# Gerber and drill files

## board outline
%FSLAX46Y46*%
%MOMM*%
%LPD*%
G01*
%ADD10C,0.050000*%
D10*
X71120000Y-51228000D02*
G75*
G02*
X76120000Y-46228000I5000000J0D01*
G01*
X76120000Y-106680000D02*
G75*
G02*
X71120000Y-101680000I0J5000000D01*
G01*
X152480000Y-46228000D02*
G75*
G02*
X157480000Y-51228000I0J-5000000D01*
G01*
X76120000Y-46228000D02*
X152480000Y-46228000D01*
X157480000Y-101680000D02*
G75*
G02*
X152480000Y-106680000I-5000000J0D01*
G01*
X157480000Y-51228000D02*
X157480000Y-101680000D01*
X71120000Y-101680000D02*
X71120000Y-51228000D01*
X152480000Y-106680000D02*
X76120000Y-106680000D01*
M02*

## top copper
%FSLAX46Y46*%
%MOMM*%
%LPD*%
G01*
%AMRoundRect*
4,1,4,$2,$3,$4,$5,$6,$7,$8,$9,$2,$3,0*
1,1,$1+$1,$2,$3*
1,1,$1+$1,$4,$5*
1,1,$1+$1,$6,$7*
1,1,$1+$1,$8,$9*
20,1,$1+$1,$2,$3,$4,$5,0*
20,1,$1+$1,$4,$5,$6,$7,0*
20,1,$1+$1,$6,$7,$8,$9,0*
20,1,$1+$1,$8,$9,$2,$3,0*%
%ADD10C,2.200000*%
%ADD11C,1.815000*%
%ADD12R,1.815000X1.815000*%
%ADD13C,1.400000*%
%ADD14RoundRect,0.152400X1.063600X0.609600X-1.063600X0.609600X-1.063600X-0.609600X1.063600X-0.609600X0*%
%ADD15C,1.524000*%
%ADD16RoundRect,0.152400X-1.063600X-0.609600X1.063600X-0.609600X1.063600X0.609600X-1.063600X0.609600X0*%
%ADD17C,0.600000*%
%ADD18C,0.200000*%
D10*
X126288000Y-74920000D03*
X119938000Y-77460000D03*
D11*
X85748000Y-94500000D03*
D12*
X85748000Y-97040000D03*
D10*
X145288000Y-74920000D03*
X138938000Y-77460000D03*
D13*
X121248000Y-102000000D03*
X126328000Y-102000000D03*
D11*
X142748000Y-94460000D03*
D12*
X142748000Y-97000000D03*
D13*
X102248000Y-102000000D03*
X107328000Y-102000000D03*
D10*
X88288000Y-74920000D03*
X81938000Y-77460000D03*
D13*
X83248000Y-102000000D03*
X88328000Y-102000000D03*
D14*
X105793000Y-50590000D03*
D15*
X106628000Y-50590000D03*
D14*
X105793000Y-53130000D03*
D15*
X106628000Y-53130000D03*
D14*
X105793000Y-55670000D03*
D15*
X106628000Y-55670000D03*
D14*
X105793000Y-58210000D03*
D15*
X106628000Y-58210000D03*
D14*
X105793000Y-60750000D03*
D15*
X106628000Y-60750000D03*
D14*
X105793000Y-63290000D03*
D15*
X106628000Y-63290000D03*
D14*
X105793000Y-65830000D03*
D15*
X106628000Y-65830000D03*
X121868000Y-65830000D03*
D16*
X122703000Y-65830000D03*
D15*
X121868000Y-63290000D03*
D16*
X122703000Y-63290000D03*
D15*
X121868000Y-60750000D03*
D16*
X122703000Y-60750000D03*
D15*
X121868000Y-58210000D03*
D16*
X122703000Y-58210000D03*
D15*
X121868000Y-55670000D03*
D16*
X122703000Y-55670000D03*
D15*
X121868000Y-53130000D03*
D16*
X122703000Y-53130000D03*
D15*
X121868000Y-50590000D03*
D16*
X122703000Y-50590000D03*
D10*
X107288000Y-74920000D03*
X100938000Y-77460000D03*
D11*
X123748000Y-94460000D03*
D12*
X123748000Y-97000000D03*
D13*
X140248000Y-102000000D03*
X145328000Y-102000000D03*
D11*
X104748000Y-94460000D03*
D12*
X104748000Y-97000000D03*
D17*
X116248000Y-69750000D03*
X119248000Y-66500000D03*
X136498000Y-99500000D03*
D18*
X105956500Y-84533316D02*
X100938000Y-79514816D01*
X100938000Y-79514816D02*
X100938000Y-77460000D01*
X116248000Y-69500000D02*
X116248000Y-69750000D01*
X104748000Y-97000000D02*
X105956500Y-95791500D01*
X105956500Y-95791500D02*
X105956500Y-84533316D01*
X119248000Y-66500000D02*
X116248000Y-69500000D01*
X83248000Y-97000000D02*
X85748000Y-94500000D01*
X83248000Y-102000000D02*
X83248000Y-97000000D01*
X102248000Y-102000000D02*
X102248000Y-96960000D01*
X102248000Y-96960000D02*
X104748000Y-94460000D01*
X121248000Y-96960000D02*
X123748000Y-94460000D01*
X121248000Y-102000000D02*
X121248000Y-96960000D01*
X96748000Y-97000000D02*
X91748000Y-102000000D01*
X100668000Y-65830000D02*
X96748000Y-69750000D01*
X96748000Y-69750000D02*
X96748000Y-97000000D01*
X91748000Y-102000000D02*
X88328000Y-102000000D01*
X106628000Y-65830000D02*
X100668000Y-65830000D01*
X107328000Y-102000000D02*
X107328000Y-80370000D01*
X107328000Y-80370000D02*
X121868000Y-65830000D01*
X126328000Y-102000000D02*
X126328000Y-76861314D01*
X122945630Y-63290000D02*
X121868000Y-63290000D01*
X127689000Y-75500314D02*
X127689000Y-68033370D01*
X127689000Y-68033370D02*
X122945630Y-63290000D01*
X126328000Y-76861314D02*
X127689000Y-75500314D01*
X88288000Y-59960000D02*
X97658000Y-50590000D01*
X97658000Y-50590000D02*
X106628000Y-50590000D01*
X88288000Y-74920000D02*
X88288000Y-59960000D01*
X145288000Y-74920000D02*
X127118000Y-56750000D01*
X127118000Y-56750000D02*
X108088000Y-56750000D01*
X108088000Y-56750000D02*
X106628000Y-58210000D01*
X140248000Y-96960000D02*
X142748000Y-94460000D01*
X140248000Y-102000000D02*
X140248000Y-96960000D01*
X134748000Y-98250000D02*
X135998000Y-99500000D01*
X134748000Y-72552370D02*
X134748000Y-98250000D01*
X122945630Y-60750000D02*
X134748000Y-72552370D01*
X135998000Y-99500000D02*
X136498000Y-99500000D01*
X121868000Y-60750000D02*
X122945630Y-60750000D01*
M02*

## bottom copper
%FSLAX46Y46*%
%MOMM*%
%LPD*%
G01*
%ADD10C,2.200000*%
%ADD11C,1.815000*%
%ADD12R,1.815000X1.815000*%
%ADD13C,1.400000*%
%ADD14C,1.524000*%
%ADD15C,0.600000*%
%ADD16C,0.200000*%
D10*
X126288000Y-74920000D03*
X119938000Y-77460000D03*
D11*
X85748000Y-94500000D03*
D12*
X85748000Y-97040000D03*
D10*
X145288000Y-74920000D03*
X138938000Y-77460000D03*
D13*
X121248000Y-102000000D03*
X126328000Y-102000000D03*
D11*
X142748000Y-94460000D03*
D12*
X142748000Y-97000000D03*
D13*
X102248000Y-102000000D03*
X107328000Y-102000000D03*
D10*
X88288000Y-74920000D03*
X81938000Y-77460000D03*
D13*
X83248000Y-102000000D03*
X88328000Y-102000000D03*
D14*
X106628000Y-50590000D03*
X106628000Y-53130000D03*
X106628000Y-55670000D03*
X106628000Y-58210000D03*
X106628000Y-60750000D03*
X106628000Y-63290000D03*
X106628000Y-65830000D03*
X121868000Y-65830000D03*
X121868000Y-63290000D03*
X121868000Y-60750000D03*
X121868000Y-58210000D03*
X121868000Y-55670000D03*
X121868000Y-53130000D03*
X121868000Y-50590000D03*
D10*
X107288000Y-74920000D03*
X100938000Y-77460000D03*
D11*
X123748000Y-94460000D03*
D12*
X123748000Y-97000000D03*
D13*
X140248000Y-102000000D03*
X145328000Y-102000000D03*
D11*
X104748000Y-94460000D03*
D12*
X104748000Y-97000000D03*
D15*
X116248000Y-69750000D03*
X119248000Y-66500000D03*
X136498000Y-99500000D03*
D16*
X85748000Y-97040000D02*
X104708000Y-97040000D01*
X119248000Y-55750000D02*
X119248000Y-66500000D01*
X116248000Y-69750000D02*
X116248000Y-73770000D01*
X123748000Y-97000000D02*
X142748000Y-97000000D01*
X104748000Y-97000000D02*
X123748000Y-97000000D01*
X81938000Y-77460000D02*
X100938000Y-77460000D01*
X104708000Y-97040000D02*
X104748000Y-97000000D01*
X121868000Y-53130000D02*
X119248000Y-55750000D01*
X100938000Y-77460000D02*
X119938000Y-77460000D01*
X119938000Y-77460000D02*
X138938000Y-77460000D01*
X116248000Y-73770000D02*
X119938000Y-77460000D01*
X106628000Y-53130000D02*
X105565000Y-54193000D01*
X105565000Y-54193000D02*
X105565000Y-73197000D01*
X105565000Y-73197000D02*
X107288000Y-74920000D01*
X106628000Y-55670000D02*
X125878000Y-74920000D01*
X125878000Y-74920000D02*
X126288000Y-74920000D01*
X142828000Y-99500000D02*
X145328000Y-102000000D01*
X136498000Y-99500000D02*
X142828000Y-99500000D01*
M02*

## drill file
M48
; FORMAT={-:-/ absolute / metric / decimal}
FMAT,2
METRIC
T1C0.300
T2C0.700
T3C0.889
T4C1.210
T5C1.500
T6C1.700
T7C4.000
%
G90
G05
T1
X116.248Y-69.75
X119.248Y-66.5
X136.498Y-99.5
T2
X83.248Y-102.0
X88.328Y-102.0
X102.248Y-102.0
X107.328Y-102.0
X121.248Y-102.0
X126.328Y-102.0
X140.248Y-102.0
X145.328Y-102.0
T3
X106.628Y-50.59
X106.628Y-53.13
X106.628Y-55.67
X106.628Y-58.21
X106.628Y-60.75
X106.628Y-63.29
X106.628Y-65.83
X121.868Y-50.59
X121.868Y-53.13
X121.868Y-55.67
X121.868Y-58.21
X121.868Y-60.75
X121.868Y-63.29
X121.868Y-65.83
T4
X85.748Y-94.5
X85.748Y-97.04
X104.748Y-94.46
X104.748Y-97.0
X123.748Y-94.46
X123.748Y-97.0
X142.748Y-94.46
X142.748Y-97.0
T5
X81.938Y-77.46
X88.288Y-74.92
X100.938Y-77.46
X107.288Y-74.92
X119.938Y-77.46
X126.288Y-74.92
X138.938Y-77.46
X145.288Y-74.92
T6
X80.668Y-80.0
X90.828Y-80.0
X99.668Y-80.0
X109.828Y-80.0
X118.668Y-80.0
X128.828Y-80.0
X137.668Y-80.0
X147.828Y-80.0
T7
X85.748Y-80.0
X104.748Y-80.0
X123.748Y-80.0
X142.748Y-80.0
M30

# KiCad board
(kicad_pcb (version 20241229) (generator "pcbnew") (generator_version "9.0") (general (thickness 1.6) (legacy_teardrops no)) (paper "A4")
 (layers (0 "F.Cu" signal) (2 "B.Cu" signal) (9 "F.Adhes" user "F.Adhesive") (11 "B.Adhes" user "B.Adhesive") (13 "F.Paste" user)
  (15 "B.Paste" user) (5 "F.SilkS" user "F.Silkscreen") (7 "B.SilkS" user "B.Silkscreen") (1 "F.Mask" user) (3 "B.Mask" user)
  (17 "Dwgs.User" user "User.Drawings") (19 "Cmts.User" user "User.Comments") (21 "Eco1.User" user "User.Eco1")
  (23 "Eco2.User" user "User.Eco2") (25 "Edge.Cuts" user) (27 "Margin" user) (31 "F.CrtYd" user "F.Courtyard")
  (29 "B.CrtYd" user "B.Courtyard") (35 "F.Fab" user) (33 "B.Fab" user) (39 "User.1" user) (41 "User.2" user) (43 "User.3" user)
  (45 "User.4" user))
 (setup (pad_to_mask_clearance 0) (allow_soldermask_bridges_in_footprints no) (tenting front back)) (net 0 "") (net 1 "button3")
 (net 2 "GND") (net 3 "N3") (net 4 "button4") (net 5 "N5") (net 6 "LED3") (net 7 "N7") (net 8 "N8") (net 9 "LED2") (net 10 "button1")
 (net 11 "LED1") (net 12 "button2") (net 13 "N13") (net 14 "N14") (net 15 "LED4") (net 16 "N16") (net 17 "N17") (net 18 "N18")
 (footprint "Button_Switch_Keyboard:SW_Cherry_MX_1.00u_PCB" (layer "F.Cu") (at 126.288 74.92)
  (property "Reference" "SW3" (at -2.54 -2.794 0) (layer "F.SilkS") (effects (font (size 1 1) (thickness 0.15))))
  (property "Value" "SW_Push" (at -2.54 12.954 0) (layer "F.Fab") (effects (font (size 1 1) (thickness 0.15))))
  (pad "" np_thru_hole circle (at -7.62 5.08) (size 1.7 1.7) (drill 1.7) (layers "*.Cu" "*.Mask"))
  (pad "" np_thru_hole circle (at -2.54 5.08) (size 4 4) (drill 4) (layers "*.Cu" "*.Mask"))
  (pad "" np_thru_hole circle (at 2.54 5.08) (size 1.7 1.7) (drill 1.7) (layers "*.Cu" "*.Mask"))
  (pad "1" thru_hole circle (at 0 0) (size 2.2 2.2) (drill 1.5) (layers "*.Cu" "*.Mask") (remove_unused_layers no) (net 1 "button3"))
  (pad "2" thru_hole circle (at -6.35 2.54) (size 2.2 2.2) (drill 1.5) (layers "*.Cu" "*.Mask") (remove_unused_layers no) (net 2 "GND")))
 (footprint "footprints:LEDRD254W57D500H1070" (layer "F.Cu") (at 85.748 95.77 90)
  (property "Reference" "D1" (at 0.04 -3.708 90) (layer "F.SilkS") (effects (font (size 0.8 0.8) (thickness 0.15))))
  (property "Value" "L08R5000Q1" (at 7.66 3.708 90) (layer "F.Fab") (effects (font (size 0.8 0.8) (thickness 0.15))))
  (pad "A" thru_hole circle (at 1.27 0 90) (size 1.815 1.815) (drill 1.21) (layers "*.Cu" "*.Mask") (remove_unused_layers no) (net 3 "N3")
   (solder_mask_margin 0.102))
  (pad "C" thru_hole rect (at -1.27 0 90) (size 1.815 1.815) (drill 1.21) (layers "*.Cu" "*.Mask") (remove_unused_layers no) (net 2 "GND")
   (solder_mask_margin 0.102)))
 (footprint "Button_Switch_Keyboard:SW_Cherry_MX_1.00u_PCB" (layer "F.Cu") (at 145.288 74.92)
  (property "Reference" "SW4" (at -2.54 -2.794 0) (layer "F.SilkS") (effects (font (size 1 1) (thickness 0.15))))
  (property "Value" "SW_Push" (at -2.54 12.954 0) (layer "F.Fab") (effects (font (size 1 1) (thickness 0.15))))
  (pad "" np_thru_hole circle (at -7.62 5.08) (size 1.7 1.7) (drill 1.7) (layers "*.Cu" "*.Mask"))
  (pad "" np_thru_hole circle (at -2.54 5.08) (size 4 4) (drill 4) (layers "*.Cu" "*.Mask"))
  (pad "" np_thru_hole circle (at 2.54 5.08) (size 1.7 1.7) (drill 1.7) (layers "*.Cu" "*.Mask"))
  (pad "1" thru_hole circle (at 0 0) (size 2.2 2.2) (drill 1.5) (layers "*.Cu" "*.Mask") (remove_unused_layers no) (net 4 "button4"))
  (pad "2" thru_hole circle (at -6.35 2.54) (size 2.2 2.2) (drill 1.5) (layers "*.Cu" "*.Mask") (remove_unused_layers no) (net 2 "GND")))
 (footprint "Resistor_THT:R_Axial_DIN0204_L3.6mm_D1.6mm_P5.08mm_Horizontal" (layer "F.Cu") (at 121.248 102)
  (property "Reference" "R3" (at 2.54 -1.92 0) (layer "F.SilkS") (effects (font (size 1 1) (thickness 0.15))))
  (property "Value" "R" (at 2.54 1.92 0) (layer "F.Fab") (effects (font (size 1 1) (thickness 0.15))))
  (pad "1" thru_hole circle (at 0 0) (size 1.4 1.4) (drill 0.7) (layers "*.Cu" "*.Mask") (remove_unused_layers no) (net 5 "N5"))
  (pad "2" thru_hole circle (at 5.08 0) (size 1.4 1.4) (drill 0.7) (layers "*.Cu" "*.Mask") (remove_unused_layers no) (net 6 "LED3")))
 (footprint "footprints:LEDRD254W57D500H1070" (layer "F.Cu") (at 142.748 95.73 90)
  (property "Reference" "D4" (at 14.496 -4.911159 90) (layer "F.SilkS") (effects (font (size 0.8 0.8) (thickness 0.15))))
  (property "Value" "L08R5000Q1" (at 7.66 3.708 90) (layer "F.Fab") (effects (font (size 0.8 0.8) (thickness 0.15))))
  (pad "A" thru_hole circle (at 1.27 0 90) (size 1.815 1.815) (drill 1.21) (layers "*.Cu" "*.Mask") (remove_unused_layers no) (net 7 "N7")
   (solder_mask_margin 0.102))
  (pad "C" thru_hole rect (at -1.27 0 90) (size 1.815 1.815) (drill 1.21) (layers "*.Cu" "*.Mask") (remove_unused_layers no) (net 2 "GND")
   (solder_mask_margin 0.102)))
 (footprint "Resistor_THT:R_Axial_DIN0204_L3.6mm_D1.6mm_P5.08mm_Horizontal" (layer "F.Cu") (at 102.248 102)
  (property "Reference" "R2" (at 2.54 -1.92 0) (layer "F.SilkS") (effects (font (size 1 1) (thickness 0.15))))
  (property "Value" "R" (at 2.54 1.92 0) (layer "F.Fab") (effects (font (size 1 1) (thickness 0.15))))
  (pad "1" thru_hole circle (at 0 0) (size 1.4 1.4) (drill 0.7) (layers "*.Cu" "*.Mask") (remove_unused_layers no) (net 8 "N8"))
  (pad "2" thru_hole circle (at 5.08 0) (size 1.4 1.4) (drill 0.7) (layers "*.Cu" "*.Mask") (remove_unused_layers no) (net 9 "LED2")))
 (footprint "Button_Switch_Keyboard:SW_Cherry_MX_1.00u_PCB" (layer "F.Cu") (at 88.288 74.92)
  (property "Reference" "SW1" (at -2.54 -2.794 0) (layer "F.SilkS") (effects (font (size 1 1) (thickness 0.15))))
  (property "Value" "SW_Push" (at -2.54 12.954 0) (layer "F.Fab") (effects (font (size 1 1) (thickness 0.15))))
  (pad "" np_thru_hole circle (at -7.62 5.08) (size 1.7 1.7) (drill 1.7) (layers "*.Cu" "*.Mask"))
  (pad "" np_thru_hole circle (at -2.54 5.08) (size 4 4) (drill 4) (layers "*.Cu" "*.Mask"))
  (pad "" np_thru_hole circle (at 2.54 5.08) (size 1.7 1.7) (drill 1.7) (layers "*.Cu" "*.Mask"))
  (pad "1" thru_hole circle (at 0 0) (size 2.2 2.2) (drill 1.5) (layers "*.Cu" "*.Mask") (remove_unused_layers no) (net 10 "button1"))
  (pad "2" thru_hole circle (at -6.35 2.54) (size 2.2 2.2) (drill 1.5) (layers "*.Cu" "*.Mask") (remove_unused_layers no) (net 2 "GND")))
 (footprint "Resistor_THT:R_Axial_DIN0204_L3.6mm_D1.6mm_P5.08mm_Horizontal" (layer "F.Cu") (at 83.248 102)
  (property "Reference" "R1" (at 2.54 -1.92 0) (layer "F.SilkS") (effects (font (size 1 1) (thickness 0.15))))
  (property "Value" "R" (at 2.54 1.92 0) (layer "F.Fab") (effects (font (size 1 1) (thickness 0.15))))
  (pad "1" thru_hole circle (at 0 0) (size 1.4 1.4) (drill 0.7) (layers "*.Cu" "*.Mask") (remove_unused_layers no) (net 3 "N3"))
  (pad "2" thru_hole circle (at 5.08 0) (size 1.4 1.4) (drill 0.7) (layers "*.Cu" "*.Mask") (remove_unused_layers no) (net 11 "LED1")))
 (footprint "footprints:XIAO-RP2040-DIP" (layer "F.Cu") (at 114.248 58.21)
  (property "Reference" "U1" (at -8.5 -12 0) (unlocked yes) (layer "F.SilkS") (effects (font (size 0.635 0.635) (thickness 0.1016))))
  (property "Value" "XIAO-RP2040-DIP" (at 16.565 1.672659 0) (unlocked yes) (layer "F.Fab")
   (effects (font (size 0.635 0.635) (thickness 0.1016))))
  (pad "1" smd roundrect (at -8.455 -7.62 180) (size 2.432 1.524) (layers "F.Cu" "F.Mask") (roundrect_rratio 0.1) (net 10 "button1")
   (thermal_bridge_angle 45))
  (pad "1" thru_hole circle (at -7.62 -7.62 180) (size 1.524 1.524) (drill 0.889) (layers "*.Cu" "*.Mask") (remove_unused_layers no)
   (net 10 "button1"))
  (pad "2" smd roundrect (at -8.455 -5.08 180) (size 2.432 1.524) (layers "F.Cu" "F.Mask") (roundrect_rratio 0.1) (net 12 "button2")
   (thermal_bridge_angle 45))
  (pad "2" thru_hole circle (at -7.62 -5.08 180) (size 1.524 1.524) (drill 0.889) (layers "*.Cu" "*.Mask") (remove_unused_layers no)
   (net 12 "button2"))
  (pad "3" smd roundrect (at -8.455 -2.54 180) (size 2.432 1.524) (layers "F.Cu" "F.Mask") (roundrect_rratio 0.1) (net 1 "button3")
   (thermal_bridge_angle 45))
  (pad "3" thru_hole circle (at -7.62 -2.54 180) (size 1.524 1.524) (drill 0.889) (layers "*.Cu" "*.Mask") (remove_unused_layers no)
   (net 1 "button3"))
  (pad "4" smd roundrect (at -8.455 0 180) (size 2.432 1.524) (layers "F.Cu" "F.Mask") (roundrect_rratio 0.1) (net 4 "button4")
   (thermal_bridge_angle 45))
  (pad "4" thru_hole circle (at -7.62 0 180) (size 1.524 1.524) (drill 0.889) (layers "*.Cu" "*.Mask") (remove_unused_layers no)
   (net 4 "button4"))
  (pad "5" smd roundrect (at -8.455 2.54 180) (size 2.432 1.524) (layers "F.Cu" "F.Mask") (roundrect_rratio 0.1) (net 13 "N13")
   (thermal_bridge_angle 45))
  (pad "5" thru_hole circle (at -7.62 2.54 180) (size 1.524 1.524) (drill 0.889) (layers "*.Cu" "*.Mask") (remove_unused_layers no)
   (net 13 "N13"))
  (pad "6" smd roundrect (at -8.455 5.08 180) (size 2.432 1.524) (layers "F.Cu" "F.Mask") (roundrect_rratio 0.1) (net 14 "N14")
   (thermal_bridge_angle 45))
  (pad "6" thru_hole circle (at -7.62 5.08 180) (size 1.524 1.524) (drill 0.889) (layers "*.Cu" "*.Mask") (remove_unused_layers no)
   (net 14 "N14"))
  (pad "7" smd roundrect (at -8.455 7.62 180) (size 2.432 1.524) (layers "F.Cu" "F.Mask") (roundrect_rratio 0.1) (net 11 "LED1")
   (thermal_bridge_angle 45))
  (pad "7" thru_hole circle (at -7.62 7.62 180) (size 1.524 1.524) (drill 0.889) (layers "*.Cu" "*.Mask") (remove_unused_layers no)
   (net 11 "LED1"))
  (pad "8" thru_hole circle (at 7.62 7.62) (size 1.524 1.524) (drill 0.889) (layers "*.Cu" "*.Mask") (remove_unused_layers no)
   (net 9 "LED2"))
  (pad "8" smd roundrect (at 8.455 7.62) (size 2.432 1.524) (layers "F.Cu" "F.Mask") (roundrect_rratio 0.1) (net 9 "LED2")
   (thermal_bridge_angle 45))
  (pad "9" thru_hole circle (at 7.62 5.08) (size 1.524 1.524) (drill 0.889) (layers "*.Cu" "*.Mask") (remove_unused_layers no)
   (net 6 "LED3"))
  (pad "9" smd roundrect (at 8.455 5.08) (size 2.432 1.524) (layers "F.Cu" "F.Mask") (roundrect_rratio 0.1) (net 6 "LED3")
   (thermal_bridge_angle 45))
  (pad "10" thru_hole circle (at 7.62 2.54) (size 1.524 1.524) (drill 0.889) (layers "*.Cu" "*.Mask") (remove_unused_layers no)
   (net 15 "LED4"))
  (pad "10" smd roundrect (at 8.455 2.54) (size 2.432 1.524) (layers "F.Cu" "F.Mask") (roundrect_rratio 0.1) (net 15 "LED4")
   (thermal_bridge_angle 45))
  (pad "11" thru_hole circle (at 7.62 0) (size 1.524 1.524) (drill 0.889) (layers "*.Cu" "*.Mask") (remove_unused_layers no) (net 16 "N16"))
  (pad "11" smd roundrect (at 8.455 0) (size 2.432 1.524) (layers "F.Cu" "F.Mask") (roundrect_rratio 0.1) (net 16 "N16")
   (thermal_bridge_angle 45))
  (pad "12" thru_hole circle (at 7.62 -2.54) (size 1.524 1.524) (drill 0.889) (layers "*.Cu" "*.Mask") (remove_unused_layers no)
   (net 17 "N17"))
  (pad "12" smd roundrect (at 8.455 -2.54) (size 2.432 1.524) (layers "F.Cu" "F.Mask") (roundrect_rratio 0.1) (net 17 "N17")
   (thermal_bridge_angle 45))
  (pad "13" thru_hole circle (at 7.62 -5.08) (size 1.524 1.524) (drill 0.889) (layers "*.Cu" "*.Mask") (remove_unused_layers no)
   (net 2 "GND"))
  (pad "13" smd roundrect (at 8.455 -5.08) (size 2.432 1.524) (layers "F.Cu" "F.Mask") (roundrect_rratio 0.1) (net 2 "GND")
   (thermal_bridge_angle 45))
  (pad "14" thru_hole circle (at 7.62 -7.62) (size 1.524 1.524) (drill 0.889) (layers "*.Cu" "*.Mask") (remove_unused_layers no)
   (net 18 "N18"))
  (pad "14" smd roundrect (at 8.455 -7.62) (size 2.432 1.524) (layers "F.Cu" "F.Mask") (roundrect_rratio 0.1) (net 18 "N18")
   (thermal_bridge_angle 45)))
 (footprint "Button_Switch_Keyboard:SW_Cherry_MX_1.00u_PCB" (layer "F.Cu") (at 107.288 74.92)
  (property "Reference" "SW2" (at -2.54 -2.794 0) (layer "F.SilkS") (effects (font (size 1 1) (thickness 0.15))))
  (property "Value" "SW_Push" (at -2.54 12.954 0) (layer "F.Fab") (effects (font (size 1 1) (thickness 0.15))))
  (pad "" np_thru_hole circle (at -7.62 5.08) (size 1.7 1.7) (drill 1.7) (layers "*.Cu" "*.Mask"))
  (pad "" np_thru_hole circle (at -2.54 5.08) (size 4 4) (drill 4) (layers "*.Cu" "*.Mask"))
  (pad "" np_thru_hole circle (at 2.54 5.08) (size 1.7 1.7) (drill 1.7) (layers "*.Cu" "*.Mask"))
  (pad "1" thru_hole circle (at 0 0) (size 2.2 2.2) (drill 1.5) (layers "*.Cu" "*.Mask") (remove_unused_layers no) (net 12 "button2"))
  (pad "2" thru_hole circle (at -6.35 2.54) (size 2.2 2.2) (drill 1.5) (layers "*.Cu" "*.Mask") (remove_unused_layers no) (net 2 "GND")))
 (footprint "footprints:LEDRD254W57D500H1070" (layer "F.Cu") (at 123.748 95.73 90)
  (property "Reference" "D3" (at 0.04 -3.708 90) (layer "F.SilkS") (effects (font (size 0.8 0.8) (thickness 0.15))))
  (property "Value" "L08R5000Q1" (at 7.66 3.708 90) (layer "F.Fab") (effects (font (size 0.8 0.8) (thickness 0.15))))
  (pad "A" thru_hole circle (at 1.27 0 90) (size 1.815 1.815) (drill 1.21) (layers "*.Cu" "*.Mask") (remove_unused_layers no) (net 5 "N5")
   (solder_mask_margin 0.102))
  (pad "C" thru_hole rect (at -1.27 0 90) (size 1.815 1.815) (drill 1.21) (layers "*.Cu" "*.Mask") (remove_unused_layers no) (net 2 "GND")
   (solder_mask_margin 0.102)))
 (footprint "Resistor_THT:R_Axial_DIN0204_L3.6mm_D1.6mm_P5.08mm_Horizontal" (layer "F.Cu") (at 140.248 102)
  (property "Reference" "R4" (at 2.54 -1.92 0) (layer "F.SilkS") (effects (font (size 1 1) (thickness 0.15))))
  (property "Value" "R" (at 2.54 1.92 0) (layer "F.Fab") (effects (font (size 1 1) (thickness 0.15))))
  (pad "1" thru_hole circle (at 0 0) (size 1.4 1.4) (drill 0.7) (layers "*.Cu" "*.Mask") (remove_unused_layers no) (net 7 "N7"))
  (pad "2" thru_hole circle (at 5.08 0) (size 1.4 1.4) (drill 0.7) (layers "*.Cu" "*.Mask") (remove_unused_layers no) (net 15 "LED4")))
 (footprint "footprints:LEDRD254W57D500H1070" (layer "F.Cu") (at 104.748 95.73 90)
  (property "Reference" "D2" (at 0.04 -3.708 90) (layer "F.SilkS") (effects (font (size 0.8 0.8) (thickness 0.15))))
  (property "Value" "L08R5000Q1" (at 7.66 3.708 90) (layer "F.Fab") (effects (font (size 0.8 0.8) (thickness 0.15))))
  (pad "A" thru_hole circle (at 1.27 0 90) (size 1.815 1.815) (drill 1.21) (layers "*.Cu" "*.Mask") (remove_unused_layers no) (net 8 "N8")
   (solder_mask_margin 0.102))
  (pad "C" thru_hole rect (at -1.27 0 90) (size 1.815 1.815) (drill 1.21) (layers "*.Cu" "*.Mask") (remove_unused_layers no) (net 2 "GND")
   (solder_mask_margin 0.102)))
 (gr_arc (start 71.12 51.228) (mid 72.584466 47.692466) (end 76.12 46.228) (stroke (width 0.05) (type default)) (layer "Edge.Cuts"))
 (gr_arc (start 76.12 106.68) (mid 72.584466 105.215534) (end 71.12 101.68) (stroke (width 0.05) (type default)) (layer "Edge.Cuts"))
 (gr_arc (start 152.48 46.228) (mid 156.015534 47.692466) (end 157.48 51.228) (stroke (width 0.05) (type default)) (layer "Edge.Cuts"))
 (gr_line (start 76.12 46.228) (end 152.48 46.228) (stroke (width 0.05) (type default)) (layer "Edge.Cuts"))
 (gr_arc (start 157.48 101.68) (mid 156.015534 105.215534) (end 152.48 106.68) (stroke (width 0.05) (type default)) (layer "Edge.Cuts"))
 (gr_line (start 157.48 51.228) (end 157.48 101.68) (stroke (width 0.05) (type default)) (layer "Edge.Cuts"))
 (gr_line (start 71.12 101.68) (end 71.12 51.228) (stroke (width 0.05) (type default)) (layer "Edge.Cuts"))
 (gr_line (start 152.48 106.68) (end 76.12 106.68) (stroke (width 0.05) (type default)) (layer "Edge.Cuts"))
 (segment (start 105.9565 84.533316) (end 100.938 79.514816) (width 0.2) (layer "F.Cu") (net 2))
 (segment (start 100.938 79.514816) (end 100.938 77.46) (width 0.2) (layer "F.Cu") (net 2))
 (segment (start 116.248 69.5) (end 116.248 69.75) (width 0.2) (layer "F.Cu") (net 2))
 (segment (start 104.748 97) (end 105.9565 95.7915) (width 0.2) (layer "F.Cu") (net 2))
 (segment (start 105.9565 95.7915) (end 105.9565 84.533316) (width 0.2) (layer "F.Cu") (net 2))
 (segment (start 119.248 66.5) (end 116.248 69.5) (width 0.2) (layer "F.Cu") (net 2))
 (via (at 116.248 69.75) (size 0.6) (drill 0.3) (layers "F.Cu" "B.Cu") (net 2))
 (via (at 119.248 66.5) (size 0.6) (drill 0.3) (layers "F.Cu" "B.Cu") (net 2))
 (segment (start 85.748 97.04) (end 104.708 97.04) (width 0.2) (layer "B.Cu") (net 2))
 (segment (start 119.248 55.75) (end 119.248 66.5) (width 0.2) (layer "B.Cu") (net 2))
 (segment (start 116.248 69.75) (end 116.248 73.77) (width 0.2) (layer "B.Cu") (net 2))
 (segment (start 123.748 97) (end 142.748 97) (width 0.2) (layer "B.Cu") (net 2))
 (segment (start 104.748 97) (end 123.748 97) (width 0.2) (layer "B.Cu") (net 2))
 (segment (start 81.938 77.46) (end 100.938 77.46) (width 0.2) (layer "B.Cu") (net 2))
 (segment (start 104.708 97.04) (end 104.748 97) (width 0.2) (layer "B.Cu") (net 2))
 (segment (start 121.868 53.13) (end 119.248 55.75) (width 0.2) (layer "B.Cu") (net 2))
 (segment (start 100.938 77.46) (end 119.938 77.46) (width 0.2) (layer "B.Cu") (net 2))
 (segment (start 119.938 77.46) (end 138.938 77.46) (width 0.2) (layer "B.Cu") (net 2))
 (segment (start 116.248 73.77) (end 119.938 77.46) (width 0.2) (layer "B.Cu") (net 2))
 (segment (start 83.248 97) (end 85.748 94.5) (width 0.2) (layer "F.Cu") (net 3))
 (segment (start 83.248 102) (end 83.248 97) (width 0.2) (layer "F.Cu") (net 3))
 (segment (start 102.248 102) (end 102.248 96.96) (width 0.2) (layer "F.Cu") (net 8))
 (segment (start 102.248 96.96) (end 104.748 94.46) (width 0.2) (layer "F.Cu") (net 8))
 (segment (start 121.248 96.96) (end 123.748 94.46) (width 0.2) (layer "F.Cu") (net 5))
 (segment (start 121.248 102) (end 121.248 96.96) (width 0.2) (layer "F.Cu") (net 5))
 (segment (start 96.748 97) (end 91.748 102) (width 0.2) (layer "F.Cu") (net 11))
 (segment (start 100.668 65.83) (end 96.748 69.75) (width 0.2) (layer "F.Cu") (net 11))
 (segment (start 96.748 69.75) (end 96.748 97) (width 0.2) (layer "F.Cu") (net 11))
 (segment (start 91.748 102) (end 88.328 102) (width 0.2) (layer "F.Cu") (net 11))
 (segment (start 106.628 65.83) (end 100.668 65.83) (width 0.2) (layer "F.Cu") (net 11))
 (segment (start 107.328 102) (end 107.328 80.37) (width 0.2) (layer "F.Cu") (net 9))
 (segment (start 107.328 80.37) (end 121.868 65.83) (width 0.2) (layer "F.Cu") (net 9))
 (segment (start 126.328 102) (end 126.328 76.861314) (width 0.2) (layer "F.Cu") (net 6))
 (segment (start 122.94563 63.29) (end 121.868 63.29) (width 0.2) (layer "F.Cu") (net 6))
 (segment (start 127.689 75.500314) (end 127.689 68.03337) (width 0.2) (layer "F.Cu") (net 6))
 (segment (start 127.689 68.03337) (end 122.94563 63.29) (width 0.2) (layer "F.Cu") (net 6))
 (segment (start 126.328 76.861314) (end 127.689 75.500314) (width 0.2) (layer "F.Cu") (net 6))
 (segment (start 88.288 59.96) (end 97.658 50.59) (width 0.2) (layer "F.Cu") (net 10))
 (segment (start 97.658 50.59) (end 106.628 50.59) (width 0.2) (layer "F.Cu") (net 10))
 (segment (start 88.288 74.92) (end 88.288 59.96) (width 0.2) (layer "F.Cu") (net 10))
 (segment (start 106.628 53.13) (end 105.565 54.193) (width 0.2) (layer "B.Cu") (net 12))
 (segment (start 105.565 54.193) (end 105.565 73.197) (width 0.2) (layer "B.Cu") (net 12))
 (segment (start 105.565 73.197) (end 107.288 74.92) (width 0.2) (layer "B.Cu") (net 12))
 (segment (start 106.628 55.67) (end 125.878 74.92) (width 0.2) (layer "B.Cu") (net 1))
 (segment (start 125.878 74.92) (end 126.288 74.92) (width 0.2) (layer "B.Cu") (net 1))
 (segment (start 145.288 74.92) (end 127.118 56.75) (width 0.2) (layer "F.Cu") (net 4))
 (segment (start 127.118 56.75) (end 108.088 56.75) (width 0.2) (layer "F.Cu") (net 4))
 (segment (start 108.088 56.75) (end 106.628 58.21) (width 0.2) (layer "F.Cu") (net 4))
 (segment (start 140.248 96.96) (end 142.748 94.46) (width 0.2) (layer "F.Cu") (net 7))
 (segment (start 140.248 102) (end 140.248 96.96) (width 0.2) (layer "F.Cu") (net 7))
 (segment (start 134.748 98.25) (end 135.998 99.5) (width 0.2) (layer "F.Cu") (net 15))
 (segment (start 134.748 72.55237) (end 134.748 98.25) (width 0.2) (layer "F.Cu") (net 15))
 (segment (start 122.94563 60.75) (end 134.748 72.55237) (width 0.2) (layer "F.Cu") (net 15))
 (segment (start 135.998 99.5) (end 136.498 99.5) (width 0.2) (layer "F.Cu") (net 15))
 (segment (start 121.868 60.75) (end 122.94563 60.75) (width 0.2) (layer "F.Cu") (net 15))
 (via (at 136.498 99.5) (size 0.6) (drill 0.3) (layers "F.Cu" "B.Cu") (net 15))
 (segment (start 142.828 99.5) (end 145.328 102) (width 0.2) (layer "B.Cu") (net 15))
 (segment (start 136.498 99.5) (end 142.828 99.5) (width 0.2) (layer "B.Cu") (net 15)))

